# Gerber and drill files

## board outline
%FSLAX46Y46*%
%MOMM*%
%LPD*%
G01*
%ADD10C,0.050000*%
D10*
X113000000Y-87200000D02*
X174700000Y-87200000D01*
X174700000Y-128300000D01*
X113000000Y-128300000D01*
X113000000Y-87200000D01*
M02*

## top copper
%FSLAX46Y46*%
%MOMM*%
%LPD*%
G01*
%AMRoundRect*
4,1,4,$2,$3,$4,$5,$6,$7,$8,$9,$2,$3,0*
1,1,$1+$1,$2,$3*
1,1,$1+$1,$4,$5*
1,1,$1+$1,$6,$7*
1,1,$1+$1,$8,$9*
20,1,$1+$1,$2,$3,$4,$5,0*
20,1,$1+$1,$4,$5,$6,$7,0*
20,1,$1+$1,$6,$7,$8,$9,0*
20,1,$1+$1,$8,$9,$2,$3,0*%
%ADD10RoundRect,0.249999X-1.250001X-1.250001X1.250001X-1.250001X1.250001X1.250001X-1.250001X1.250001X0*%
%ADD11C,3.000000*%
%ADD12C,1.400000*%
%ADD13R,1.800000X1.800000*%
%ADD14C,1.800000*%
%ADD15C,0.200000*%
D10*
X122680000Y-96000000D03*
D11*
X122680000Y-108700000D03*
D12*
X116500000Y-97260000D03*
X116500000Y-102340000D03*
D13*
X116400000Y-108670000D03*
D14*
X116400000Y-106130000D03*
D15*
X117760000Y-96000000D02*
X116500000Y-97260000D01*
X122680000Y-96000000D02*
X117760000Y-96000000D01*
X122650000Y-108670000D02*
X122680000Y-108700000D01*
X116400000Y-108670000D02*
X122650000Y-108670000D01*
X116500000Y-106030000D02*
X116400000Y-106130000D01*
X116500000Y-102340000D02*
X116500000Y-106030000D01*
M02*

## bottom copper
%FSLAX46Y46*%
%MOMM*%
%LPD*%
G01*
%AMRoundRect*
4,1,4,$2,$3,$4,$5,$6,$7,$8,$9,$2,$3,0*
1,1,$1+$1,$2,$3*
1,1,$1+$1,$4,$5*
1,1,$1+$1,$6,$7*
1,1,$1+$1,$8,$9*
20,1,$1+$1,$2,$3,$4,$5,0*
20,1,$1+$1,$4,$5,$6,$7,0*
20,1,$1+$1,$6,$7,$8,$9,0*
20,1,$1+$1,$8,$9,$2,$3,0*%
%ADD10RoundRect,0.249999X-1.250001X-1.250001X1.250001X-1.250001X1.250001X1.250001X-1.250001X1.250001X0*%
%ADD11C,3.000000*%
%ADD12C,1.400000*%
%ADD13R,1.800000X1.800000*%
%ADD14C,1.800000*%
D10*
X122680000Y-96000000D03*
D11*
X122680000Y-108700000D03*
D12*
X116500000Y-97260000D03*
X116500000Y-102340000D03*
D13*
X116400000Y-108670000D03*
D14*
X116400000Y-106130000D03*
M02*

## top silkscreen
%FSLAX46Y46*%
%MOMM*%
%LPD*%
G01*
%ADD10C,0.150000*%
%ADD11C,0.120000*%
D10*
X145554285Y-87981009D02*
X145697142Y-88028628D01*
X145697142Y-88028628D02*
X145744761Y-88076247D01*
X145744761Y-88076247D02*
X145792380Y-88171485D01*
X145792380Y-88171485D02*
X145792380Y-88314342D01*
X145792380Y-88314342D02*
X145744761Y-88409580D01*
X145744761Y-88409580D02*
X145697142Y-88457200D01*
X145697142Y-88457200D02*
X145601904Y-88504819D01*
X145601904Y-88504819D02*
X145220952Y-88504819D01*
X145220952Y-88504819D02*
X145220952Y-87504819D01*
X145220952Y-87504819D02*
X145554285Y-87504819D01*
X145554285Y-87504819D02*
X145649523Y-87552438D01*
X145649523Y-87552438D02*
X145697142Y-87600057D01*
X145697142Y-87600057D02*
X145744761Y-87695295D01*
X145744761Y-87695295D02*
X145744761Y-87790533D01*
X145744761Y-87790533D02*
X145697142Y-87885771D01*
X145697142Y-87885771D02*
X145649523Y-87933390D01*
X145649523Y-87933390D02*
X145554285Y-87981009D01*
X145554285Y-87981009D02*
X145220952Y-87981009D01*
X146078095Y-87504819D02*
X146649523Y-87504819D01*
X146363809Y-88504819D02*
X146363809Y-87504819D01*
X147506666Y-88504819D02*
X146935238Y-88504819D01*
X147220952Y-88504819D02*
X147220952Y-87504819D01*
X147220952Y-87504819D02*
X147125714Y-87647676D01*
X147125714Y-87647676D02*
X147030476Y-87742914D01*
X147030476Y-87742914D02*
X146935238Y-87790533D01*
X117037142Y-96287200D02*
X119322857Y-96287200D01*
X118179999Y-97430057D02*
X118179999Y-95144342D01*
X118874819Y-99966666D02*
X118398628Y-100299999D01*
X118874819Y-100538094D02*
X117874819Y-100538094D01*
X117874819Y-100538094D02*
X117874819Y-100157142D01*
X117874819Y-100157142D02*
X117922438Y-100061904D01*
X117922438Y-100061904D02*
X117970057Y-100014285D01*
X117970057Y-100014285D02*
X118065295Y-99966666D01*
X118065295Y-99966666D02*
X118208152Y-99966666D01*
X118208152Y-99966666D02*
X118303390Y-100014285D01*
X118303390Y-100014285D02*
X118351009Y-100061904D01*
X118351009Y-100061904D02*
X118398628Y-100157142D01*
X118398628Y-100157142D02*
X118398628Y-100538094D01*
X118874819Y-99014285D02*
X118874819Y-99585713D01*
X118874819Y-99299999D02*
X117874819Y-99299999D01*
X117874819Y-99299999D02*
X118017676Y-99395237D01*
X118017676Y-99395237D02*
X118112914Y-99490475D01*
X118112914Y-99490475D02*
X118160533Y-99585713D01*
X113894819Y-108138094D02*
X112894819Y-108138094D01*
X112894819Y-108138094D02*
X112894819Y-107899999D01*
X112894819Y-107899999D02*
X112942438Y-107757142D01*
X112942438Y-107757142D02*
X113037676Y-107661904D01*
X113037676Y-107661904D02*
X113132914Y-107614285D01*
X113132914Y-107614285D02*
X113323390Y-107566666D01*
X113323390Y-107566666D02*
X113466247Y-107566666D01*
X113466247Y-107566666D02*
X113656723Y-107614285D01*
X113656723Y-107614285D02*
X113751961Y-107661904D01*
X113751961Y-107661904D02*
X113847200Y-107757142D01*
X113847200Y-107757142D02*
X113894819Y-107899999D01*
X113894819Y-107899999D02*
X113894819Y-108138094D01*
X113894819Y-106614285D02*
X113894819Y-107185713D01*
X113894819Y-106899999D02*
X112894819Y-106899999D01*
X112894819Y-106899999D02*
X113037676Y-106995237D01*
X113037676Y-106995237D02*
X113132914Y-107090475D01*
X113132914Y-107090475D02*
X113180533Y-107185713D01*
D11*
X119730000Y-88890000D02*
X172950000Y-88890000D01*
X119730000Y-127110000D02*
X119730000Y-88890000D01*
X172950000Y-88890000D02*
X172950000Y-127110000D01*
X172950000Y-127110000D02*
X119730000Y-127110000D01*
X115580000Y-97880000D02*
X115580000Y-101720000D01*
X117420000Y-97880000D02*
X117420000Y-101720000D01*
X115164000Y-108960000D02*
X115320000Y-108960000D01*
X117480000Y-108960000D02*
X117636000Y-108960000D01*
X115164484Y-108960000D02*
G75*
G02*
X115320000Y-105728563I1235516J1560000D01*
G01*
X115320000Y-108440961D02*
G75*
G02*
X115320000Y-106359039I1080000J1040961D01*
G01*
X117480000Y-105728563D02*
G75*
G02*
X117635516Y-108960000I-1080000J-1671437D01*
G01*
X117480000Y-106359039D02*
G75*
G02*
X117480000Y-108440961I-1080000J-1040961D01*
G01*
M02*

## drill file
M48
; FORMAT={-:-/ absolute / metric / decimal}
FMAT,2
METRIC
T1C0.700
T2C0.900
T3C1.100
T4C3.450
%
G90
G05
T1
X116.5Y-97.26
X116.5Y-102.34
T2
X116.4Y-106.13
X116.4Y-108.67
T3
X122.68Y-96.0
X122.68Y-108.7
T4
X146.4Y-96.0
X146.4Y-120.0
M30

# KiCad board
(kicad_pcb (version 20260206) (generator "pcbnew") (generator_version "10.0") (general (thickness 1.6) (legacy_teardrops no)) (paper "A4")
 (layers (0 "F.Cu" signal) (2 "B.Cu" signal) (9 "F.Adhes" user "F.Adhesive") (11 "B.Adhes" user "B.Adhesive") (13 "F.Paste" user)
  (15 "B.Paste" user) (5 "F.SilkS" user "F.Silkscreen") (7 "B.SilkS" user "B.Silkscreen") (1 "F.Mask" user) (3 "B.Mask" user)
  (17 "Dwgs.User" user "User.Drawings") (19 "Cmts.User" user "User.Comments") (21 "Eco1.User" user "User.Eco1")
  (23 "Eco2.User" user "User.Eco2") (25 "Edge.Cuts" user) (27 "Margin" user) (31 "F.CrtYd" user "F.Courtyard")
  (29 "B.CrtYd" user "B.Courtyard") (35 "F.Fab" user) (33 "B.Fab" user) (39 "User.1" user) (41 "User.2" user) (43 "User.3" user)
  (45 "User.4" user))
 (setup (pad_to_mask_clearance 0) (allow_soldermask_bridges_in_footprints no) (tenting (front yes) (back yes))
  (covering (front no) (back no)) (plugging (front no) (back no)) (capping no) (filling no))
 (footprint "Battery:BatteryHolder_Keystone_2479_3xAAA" (layer "F.Cu") (at 122.68 96)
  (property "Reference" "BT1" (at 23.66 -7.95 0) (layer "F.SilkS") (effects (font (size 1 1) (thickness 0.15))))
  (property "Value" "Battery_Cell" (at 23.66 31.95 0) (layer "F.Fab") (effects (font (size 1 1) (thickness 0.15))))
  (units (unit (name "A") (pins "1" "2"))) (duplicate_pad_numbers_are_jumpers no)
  (fp_line (start -2.95 -7.11) (end 50.27 -7.11) (stroke (width 0.12) (type solid)) (layer "F.SilkS"))
  (fp_line (start -2.95 31.11) (end -2.95 -7.11) (stroke (width 0.12) (type solid)) (layer "F.SilkS"))
  (fp_line (start 50.27 -7.11) (end 50.27 31.11) (stroke (width 0.12) (type solid)) (layer "F.SilkS"))
  (fp_line (start 50.27 31.11) (end -2.95 31.11) (stroke (width 0.12) (type solid)) (layer "F.SilkS"))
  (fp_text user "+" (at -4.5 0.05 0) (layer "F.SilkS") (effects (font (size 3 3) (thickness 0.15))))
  (pad "" np_thru_hole circle (at 23.72 0) (size 3.45 3.45) (drill 3.45) (layers "*.Cu" "*.Mask"))
  (pad "" np_thru_hole circle (at 23.72 24) (size 3.45 3.45) (drill 3.45) (layers "*.Cu" "*.Mask"))
  (pad "1" thru_hole roundrect (at 0 0) (size 3 3) (drill 1.1) (layers "*.Cu" "*.Mask") (remove_unused_layers no)
   (roundrect_rratio 0.083333) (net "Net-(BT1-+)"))
  (pad "2" thru_hole circle (at 0 12.7) (size 3 3) (drill 1.1) (layers "*.Cu" "*.Mask") (remove_unused_layers no) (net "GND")))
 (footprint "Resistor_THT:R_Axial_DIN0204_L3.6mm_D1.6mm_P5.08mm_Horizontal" (layer "F.Cu") (at 116.5 97.26 -90)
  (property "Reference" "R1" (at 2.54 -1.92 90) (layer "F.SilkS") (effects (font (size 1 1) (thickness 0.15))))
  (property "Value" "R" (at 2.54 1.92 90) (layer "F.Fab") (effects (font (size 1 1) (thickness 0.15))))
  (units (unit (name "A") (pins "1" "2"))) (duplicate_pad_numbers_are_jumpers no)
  (fp_line (start 0.62 0.92) (end 4.46 0.92) (stroke (width 0.12) (type solid)) (layer "F.SilkS"))
  (fp_line (start 0.62 -0.92) (end 4.46 -0.92) (stroke (width 0.12) (type solid)) (layer "F.SilkS"))
  (pad "1" thru_hole circle (at 0 0 270) (size 1.4 1.4) (drill 0.7) (layers "*.Cu" "*.Mask") (remove_unused_layers no) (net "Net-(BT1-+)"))
  (pad "2" thru_hole circle (at 5.08 0 270) (size 1.4 1.4) (drill 0.7) (layers "*.Cu" "*.Mask") (remove_unused_layers no) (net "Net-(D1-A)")))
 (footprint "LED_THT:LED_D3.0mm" (layer "F.Cu") (at 116.4 108.67 90)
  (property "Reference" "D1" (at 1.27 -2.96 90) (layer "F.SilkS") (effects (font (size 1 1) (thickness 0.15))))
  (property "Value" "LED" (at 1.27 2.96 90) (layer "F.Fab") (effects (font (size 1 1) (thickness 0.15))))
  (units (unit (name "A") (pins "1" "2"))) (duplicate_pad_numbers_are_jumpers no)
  (fp_line (start -0.29 -1.236) (end -0.29 -1.08) (stroke (width 0.12) (type solid)) (layer "F.SilkS"))
  (fp_line (start -0.29 1.08) (end -0.29 1.236) (stroke (width 0.12) (type solid)) (layer "F.SilkS"))
  (fp_arc (start -0.29 -1.235516) (mid 1.36566 -1.987699) (end 2.941437 -1.08) (stroke (width 0.12) (type solid)) (layer "F.SilkS"))
  (fp_arc (start 0.229039 -1.08) (mid 1.27 -1.5) (end 2.310961 -1.08) (stroke (width 0.12) (type solid)) (layer "F.SilkS"))
  (fp_arc (start 2.941437 1.08) (mid 1.36566 1.987699) (end -0.29 1.235516) (stroke (width 0.12) (type solid)) (layer "F.SilkS"))
  (fp_arc (start 2.310961 1.08) (mid 1.27 1.5) (end 0.229039 1.08) (stroke (width 0.12) (type solid)) (layer "F.SilkS"))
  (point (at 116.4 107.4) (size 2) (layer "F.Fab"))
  (pad "1" thru_hole rect (at 0 0 90) (size 1.8 1.8) (drill 0.9) (layers "*.Cu" "*.Mask") (remove_unused_layers no) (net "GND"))
  (pad "2" thru_hole circle (at 2.54 0 90) (size 1.8 1.8) (drill 0.9) (layers "*.Cu" "*.Mask") (remove_unused_layers no) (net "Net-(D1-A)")))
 (gr_rect (start 113 87.2) (end 174.7 128.3) (stroke (width 0.05) (type default)) (fill no) (layer "Edge.Cuts"))
 (segment (start 117.76 96) (end 116.5 97.26) (width 0.2) (layer "F.Cu") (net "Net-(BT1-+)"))
 (segment (start 122.68 96) (end 117.76 96) (width 0.2) (layer "F.Cu") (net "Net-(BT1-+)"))
 (segment (start 122.65 108.67) (end 122.68 108.7) (width 0.2) (layer "F.Cu") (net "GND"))
 (segment (start 116.4 108.67) (end 122.65 108.67) (width 0.2) (layer "F.Cu") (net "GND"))
 (segment (start 116.5 106.03) (end 116.4 106.13) (width 0.2) (layer "F.Cu") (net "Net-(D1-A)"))
 (segment (start 116.5 102.34) (end 116.5 106.03) (width 0.2) (layer "F.Cu") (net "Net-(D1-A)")))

